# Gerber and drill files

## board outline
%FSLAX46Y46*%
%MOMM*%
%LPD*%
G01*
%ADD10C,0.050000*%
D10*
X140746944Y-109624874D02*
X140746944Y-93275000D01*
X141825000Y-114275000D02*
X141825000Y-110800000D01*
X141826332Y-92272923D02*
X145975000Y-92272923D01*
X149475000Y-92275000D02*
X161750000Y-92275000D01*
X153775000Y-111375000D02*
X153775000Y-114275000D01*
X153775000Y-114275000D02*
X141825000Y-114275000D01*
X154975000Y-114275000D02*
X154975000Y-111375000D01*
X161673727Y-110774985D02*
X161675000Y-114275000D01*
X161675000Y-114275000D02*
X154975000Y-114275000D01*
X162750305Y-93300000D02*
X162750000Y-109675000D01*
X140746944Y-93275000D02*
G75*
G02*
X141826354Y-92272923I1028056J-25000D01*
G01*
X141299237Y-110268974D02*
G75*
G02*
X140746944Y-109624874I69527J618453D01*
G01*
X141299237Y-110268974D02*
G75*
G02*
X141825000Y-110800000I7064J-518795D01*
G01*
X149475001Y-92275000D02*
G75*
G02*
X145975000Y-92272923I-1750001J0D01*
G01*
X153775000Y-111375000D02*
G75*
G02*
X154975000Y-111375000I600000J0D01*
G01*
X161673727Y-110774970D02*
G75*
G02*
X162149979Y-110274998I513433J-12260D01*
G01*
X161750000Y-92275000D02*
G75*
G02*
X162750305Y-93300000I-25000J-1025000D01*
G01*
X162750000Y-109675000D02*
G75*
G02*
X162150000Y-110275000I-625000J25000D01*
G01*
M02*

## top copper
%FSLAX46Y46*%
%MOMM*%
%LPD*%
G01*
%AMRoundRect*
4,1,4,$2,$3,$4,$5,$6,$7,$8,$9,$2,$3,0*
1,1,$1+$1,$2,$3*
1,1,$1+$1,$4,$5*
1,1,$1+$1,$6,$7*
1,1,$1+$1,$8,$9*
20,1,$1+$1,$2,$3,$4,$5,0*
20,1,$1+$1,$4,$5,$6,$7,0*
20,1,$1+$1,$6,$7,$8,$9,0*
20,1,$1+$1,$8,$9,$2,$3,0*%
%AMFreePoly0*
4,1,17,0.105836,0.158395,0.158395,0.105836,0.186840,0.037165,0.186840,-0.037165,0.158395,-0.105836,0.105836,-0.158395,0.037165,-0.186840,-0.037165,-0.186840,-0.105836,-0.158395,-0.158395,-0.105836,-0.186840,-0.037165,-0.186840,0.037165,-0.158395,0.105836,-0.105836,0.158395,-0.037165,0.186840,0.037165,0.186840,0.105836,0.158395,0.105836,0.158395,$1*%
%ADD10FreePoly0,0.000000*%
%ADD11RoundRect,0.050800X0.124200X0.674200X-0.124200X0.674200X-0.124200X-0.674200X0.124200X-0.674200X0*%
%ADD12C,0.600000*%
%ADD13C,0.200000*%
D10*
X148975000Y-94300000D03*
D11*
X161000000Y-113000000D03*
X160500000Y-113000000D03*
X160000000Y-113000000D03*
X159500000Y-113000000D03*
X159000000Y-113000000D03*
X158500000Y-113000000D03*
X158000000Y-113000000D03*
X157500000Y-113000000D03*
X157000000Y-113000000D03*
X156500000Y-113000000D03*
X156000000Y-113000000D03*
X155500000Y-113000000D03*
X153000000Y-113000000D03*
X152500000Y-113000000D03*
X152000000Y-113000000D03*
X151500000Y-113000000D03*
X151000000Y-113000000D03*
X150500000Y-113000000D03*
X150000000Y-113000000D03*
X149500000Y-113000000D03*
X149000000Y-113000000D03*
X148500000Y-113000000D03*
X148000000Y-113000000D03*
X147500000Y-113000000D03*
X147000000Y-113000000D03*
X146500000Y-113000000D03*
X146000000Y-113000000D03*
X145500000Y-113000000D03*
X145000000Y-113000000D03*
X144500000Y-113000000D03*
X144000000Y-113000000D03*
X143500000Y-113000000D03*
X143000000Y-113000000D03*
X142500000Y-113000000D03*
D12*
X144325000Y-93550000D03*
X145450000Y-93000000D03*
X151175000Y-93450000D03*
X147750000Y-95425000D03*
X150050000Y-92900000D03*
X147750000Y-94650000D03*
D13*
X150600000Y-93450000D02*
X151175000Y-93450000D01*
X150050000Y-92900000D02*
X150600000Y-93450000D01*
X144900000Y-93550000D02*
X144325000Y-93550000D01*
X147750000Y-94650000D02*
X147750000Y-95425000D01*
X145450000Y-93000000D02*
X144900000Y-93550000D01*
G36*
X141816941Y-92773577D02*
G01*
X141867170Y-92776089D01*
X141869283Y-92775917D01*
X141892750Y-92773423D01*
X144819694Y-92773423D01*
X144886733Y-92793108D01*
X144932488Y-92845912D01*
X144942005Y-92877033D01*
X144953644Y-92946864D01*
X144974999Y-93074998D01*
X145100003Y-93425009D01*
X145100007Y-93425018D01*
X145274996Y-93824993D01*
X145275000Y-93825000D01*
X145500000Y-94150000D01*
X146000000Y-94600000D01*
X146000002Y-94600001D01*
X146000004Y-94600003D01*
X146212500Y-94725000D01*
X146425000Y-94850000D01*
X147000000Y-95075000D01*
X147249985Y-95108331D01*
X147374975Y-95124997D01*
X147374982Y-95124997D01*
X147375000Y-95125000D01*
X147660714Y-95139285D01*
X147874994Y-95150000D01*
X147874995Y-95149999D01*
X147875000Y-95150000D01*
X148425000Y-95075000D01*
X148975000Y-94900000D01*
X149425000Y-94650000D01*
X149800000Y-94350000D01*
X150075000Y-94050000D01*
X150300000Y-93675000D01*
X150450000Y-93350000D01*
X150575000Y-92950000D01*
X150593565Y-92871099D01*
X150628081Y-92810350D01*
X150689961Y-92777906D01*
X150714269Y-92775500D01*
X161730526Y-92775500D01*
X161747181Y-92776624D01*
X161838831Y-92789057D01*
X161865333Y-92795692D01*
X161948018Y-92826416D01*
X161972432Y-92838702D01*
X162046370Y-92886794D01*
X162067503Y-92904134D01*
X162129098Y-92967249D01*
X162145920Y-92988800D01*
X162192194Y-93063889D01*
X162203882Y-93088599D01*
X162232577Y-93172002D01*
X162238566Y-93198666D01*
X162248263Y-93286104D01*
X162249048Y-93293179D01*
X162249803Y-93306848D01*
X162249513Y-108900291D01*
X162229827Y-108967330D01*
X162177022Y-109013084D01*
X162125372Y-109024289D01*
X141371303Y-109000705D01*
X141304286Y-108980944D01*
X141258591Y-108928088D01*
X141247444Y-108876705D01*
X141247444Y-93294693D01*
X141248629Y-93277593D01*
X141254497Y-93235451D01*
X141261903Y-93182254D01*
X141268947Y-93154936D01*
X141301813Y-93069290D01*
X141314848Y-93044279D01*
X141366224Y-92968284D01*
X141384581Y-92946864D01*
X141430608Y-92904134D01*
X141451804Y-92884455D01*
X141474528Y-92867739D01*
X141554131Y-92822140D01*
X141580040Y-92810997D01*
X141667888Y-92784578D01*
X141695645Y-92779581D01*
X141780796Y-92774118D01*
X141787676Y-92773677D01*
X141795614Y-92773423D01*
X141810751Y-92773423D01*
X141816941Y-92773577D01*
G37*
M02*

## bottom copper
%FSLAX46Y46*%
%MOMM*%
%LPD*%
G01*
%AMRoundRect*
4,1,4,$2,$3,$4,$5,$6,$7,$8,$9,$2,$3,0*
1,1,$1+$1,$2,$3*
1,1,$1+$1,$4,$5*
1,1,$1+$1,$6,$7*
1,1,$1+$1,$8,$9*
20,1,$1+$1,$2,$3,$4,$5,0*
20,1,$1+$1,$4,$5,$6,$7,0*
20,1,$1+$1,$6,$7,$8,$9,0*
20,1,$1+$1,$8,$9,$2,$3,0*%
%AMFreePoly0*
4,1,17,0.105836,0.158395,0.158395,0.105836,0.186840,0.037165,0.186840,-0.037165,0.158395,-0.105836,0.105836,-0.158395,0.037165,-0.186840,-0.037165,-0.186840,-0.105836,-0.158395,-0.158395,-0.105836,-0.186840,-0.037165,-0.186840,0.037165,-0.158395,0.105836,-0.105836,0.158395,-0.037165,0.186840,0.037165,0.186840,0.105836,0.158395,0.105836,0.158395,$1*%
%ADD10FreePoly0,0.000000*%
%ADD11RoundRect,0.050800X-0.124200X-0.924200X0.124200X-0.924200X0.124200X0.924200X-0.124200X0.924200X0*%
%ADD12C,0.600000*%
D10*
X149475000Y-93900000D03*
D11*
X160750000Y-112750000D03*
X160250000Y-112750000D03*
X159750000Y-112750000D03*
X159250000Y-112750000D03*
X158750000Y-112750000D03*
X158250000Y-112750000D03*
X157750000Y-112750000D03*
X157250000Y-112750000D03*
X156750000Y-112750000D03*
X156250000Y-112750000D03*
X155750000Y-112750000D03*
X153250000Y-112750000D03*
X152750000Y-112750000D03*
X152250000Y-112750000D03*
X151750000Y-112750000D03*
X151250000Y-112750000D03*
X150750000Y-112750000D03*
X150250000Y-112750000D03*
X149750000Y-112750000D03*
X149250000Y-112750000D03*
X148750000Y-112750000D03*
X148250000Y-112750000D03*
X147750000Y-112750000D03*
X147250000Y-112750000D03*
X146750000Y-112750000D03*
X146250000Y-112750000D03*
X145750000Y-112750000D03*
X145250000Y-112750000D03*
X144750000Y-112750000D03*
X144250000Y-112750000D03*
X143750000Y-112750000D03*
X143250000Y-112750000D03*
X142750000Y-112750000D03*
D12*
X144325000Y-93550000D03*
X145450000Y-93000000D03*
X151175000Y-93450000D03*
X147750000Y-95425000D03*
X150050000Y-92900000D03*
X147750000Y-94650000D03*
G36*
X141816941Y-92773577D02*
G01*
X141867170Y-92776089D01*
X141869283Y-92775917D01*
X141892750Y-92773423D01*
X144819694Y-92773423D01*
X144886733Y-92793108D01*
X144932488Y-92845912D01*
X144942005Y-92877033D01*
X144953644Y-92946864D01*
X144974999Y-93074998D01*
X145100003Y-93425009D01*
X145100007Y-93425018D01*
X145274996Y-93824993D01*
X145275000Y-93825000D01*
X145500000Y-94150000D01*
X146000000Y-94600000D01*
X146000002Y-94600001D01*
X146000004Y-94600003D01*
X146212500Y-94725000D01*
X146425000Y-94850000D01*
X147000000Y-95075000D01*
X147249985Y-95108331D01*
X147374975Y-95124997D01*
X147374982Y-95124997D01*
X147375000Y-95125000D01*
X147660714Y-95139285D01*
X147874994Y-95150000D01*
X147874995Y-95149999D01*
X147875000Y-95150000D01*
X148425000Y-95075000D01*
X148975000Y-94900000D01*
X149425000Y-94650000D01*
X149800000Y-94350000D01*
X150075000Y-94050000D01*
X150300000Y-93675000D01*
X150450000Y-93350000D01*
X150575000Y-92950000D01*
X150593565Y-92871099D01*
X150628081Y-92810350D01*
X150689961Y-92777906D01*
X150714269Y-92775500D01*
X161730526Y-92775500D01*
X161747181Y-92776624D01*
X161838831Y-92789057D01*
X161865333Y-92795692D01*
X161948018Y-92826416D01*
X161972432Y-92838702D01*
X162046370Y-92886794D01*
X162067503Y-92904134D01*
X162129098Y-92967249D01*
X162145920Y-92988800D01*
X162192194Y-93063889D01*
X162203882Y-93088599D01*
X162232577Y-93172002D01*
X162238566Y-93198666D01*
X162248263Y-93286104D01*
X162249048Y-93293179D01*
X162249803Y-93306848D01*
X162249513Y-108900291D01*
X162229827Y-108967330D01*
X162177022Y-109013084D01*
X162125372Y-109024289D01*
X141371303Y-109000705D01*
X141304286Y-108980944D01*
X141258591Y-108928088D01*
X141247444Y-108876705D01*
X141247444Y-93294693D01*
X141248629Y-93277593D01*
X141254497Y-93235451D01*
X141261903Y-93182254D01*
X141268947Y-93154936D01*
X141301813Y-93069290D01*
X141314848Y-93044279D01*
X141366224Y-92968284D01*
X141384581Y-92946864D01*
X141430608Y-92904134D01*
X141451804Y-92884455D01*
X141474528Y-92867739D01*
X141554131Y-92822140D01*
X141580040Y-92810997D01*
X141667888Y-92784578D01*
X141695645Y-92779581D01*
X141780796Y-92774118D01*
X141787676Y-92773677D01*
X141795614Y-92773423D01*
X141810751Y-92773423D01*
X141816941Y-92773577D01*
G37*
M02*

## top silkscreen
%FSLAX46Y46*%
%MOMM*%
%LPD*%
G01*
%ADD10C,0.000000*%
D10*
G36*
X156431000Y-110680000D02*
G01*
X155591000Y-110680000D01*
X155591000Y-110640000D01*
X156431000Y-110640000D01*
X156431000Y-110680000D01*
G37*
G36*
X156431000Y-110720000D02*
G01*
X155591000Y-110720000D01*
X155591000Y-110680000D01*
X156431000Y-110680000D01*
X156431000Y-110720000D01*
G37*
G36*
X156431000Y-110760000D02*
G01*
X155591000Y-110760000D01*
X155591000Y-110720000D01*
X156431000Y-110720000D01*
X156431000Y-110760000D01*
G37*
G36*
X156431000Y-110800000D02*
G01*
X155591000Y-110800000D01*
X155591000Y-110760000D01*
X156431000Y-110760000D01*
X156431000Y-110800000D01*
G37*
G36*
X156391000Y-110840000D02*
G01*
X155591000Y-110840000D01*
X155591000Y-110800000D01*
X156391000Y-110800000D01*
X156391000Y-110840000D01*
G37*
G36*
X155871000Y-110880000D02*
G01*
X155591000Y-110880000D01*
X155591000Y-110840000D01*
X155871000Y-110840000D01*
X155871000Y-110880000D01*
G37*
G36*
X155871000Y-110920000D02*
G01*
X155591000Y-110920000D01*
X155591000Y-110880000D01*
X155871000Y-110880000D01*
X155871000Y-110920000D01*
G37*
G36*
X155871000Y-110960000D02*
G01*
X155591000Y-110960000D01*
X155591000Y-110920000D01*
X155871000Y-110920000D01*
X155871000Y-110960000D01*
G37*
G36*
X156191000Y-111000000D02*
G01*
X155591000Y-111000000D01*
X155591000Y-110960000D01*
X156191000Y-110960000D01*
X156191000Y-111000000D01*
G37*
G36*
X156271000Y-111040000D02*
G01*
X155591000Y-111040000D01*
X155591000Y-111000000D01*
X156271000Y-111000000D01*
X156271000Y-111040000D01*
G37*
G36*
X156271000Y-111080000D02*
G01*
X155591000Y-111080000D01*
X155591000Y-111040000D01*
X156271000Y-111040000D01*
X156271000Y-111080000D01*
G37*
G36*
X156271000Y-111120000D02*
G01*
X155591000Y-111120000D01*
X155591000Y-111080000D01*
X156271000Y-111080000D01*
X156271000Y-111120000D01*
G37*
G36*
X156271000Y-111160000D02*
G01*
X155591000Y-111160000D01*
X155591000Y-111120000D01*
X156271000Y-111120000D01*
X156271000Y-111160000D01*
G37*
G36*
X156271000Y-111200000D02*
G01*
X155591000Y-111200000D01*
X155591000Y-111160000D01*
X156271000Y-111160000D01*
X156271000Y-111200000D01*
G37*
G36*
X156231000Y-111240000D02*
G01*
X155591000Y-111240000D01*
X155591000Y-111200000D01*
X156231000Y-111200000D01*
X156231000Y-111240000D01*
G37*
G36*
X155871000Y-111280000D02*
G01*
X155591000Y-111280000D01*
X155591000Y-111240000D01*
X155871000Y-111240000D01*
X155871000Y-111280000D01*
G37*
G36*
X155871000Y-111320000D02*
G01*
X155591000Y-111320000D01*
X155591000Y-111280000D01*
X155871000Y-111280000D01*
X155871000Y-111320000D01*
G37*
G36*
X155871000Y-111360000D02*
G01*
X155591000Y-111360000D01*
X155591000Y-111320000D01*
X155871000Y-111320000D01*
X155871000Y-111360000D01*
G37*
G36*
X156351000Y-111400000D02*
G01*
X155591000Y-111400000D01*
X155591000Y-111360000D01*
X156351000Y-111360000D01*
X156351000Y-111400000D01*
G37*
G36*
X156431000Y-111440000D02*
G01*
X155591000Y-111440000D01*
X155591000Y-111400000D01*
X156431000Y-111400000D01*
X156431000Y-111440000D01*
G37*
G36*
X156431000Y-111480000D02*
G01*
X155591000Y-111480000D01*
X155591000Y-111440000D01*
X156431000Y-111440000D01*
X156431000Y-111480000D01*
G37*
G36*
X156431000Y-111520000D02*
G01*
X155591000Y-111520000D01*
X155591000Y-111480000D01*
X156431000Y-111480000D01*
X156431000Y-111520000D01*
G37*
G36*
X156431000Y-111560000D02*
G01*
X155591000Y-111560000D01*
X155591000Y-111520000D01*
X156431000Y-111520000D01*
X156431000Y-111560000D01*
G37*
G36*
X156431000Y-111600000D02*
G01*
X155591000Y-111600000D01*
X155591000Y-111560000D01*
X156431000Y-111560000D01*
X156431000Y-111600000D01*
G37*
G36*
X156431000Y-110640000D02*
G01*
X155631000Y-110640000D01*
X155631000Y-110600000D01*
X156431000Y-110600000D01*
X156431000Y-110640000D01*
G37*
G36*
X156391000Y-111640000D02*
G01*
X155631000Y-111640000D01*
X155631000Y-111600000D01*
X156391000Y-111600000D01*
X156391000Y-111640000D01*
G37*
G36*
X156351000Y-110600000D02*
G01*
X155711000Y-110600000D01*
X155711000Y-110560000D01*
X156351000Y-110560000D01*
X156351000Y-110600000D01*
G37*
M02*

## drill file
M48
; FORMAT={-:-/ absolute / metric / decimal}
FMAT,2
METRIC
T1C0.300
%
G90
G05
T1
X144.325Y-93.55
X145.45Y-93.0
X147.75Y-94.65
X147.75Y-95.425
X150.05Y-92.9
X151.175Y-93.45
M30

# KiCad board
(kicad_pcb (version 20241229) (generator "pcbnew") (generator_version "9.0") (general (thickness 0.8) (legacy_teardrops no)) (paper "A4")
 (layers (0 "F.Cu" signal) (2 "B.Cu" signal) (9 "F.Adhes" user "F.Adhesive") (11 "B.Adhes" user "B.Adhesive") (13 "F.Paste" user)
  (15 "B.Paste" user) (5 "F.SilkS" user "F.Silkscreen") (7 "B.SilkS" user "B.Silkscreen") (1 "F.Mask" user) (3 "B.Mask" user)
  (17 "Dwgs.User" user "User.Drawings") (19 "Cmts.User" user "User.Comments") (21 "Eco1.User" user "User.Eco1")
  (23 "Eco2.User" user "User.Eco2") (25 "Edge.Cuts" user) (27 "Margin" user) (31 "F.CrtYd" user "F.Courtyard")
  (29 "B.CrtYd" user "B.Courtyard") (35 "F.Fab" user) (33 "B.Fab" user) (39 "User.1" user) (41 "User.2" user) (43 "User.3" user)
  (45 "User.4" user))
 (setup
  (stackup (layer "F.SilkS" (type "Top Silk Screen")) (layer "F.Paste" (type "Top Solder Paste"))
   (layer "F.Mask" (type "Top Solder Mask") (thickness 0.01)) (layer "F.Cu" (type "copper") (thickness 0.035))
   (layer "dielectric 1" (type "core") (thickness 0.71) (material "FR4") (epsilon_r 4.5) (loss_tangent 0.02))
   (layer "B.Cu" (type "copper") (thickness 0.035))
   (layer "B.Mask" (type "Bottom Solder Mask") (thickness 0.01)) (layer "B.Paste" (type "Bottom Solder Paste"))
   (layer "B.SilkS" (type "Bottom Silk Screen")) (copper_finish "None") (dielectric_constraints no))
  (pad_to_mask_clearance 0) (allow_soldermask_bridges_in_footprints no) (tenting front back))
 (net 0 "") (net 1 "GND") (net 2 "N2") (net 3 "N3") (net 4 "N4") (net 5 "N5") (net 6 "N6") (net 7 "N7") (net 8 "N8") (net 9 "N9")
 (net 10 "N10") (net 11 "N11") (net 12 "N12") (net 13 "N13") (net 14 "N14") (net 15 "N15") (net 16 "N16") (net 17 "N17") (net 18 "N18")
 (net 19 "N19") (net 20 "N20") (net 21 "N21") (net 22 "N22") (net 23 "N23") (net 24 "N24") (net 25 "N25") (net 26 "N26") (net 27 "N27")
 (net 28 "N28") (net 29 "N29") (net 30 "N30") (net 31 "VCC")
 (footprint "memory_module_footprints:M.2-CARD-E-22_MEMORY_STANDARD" (layer "F.Cu") (at 151.75 114.275)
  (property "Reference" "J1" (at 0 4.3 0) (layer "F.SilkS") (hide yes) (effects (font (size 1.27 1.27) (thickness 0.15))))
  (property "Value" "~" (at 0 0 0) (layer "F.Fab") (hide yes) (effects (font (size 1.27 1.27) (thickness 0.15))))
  (fp_poly
   (pts (xy 3.841 -3.595) (xy 4.681 -3.595) (xy 4.681 -3.635) (xy 3.841 -3.635)) (stroke (width 0) (type default)) (fill yes)
   (layer "F.SilkS"))
  (fp_poly
   (pts (xy 3.841 -3.555) (xy 4.681 -3.555) (xy 4.681 -3.595) (xy 3.841 -3.595)) (stroke (width 0) (type default)) (fill yes)
   (layer "F.SilkS"))
  (fp_poly
   (pts (xy 3.841 -3.515) (xy 4.681 -3.515) (xy 4.681 -3.555) (xy 3.841 -3.555)) (stroke (width 0) (type default)) (fill yes)
   (layer "F.SilkS"))
  (fp_poly
   (pts (xy 3.841 -3.475) (xy 4.681 -3.475) (xy 4.681 -3.515) (xy 3.841 -3.515)) (stroke (width 0) (type default)) (fill yes)
   (layer "F.SilkS"))
  (fp_poly
   (pts (xy 3.841 -3.435) (xy 4.641 -3.435) (xy 4.641 -3.475) (xy 3.841 -3.475)) (stroke (width 0) (type default)) (fill yes)
   (layer "F.SilkS"))
  (fp_poly
   (pts (xy 3.841 -3.395) (xy 4.121 -3.395) (xy 4.121 -3.435) (xy 3.841 -3.435)) (stroke (width 0) (type default)) (fill yes)
   (layer "F.SilkS"))
  (fp_poly
   (pts (xy 3.841 -3.355) (xy 4.121 -3.355) (xy 4.121 -3.395) (xy 3.841 -3.395)) (stroke (width 0) (type default)) (fill yes)
   (layer "F.SilkS"))
  (fp_poly
   (pts (xy 3.841 -3.315) (xy 4.121 -3.315) (xy 4.121 -3.355) (xy 3.841 -3.355)) (stroke (width 0) (type default)) (fill yes)
   (layer "F.SilkS"))
  (fp_poly
   (pts (xy 3.841 -3.275) (xy 4.441 -3.275) (xy 4.441 -3.315) (xy 3.841 -3.315)) (stroke (width 0) (type default)) (fill yes)
   (layer "F.SilkS"))
  (fp_poly
   (pts (xy 3.841 -3.235) (xy 4.521 -3.235) (xy 4.521 -3.275) (xy 3.841 -3.275)) (stroke (width 0) (type default)) (fill yes)
   (layer "F.SilkS"))
  (fp_poly
   (pts (xy 3.841 -3.195) (xy 4.521 -3.195) (xy 4.521 -3.235) (xy 3.841 -3.235)) (stroke (width 0) (type default)) (fill yes)
   (layer "F.SilkS"))
  (fp_poly
   (pts (xy 3.841 -3.155) (xy 4.521 -3.155) (xy 4.521 -3.195) (xy 3.841 -3.195)) (stroke (width 0) (type default)) (fill yes)
   (layer "F.SilkS"))
  (fp_poly
   (pts (xy 3.841 -3.115) (xy 4.521 -3.115) (xy 4.521 -3.155) (xy 3.841 -3.155)) (stroke (width 0) (type default)) (fill yes)
   (layer "F.SilkS"))
  (fp_poly
   (pts (xy 3.841 -3.075) (xy 4.521 -3.075) (xy 4.521 -3.115) (xy 3.841 -3.115)) (stroke (width 0) (type default)) (fill yes)
   (layer "F.SilkS"))
  (fp_poly
   (pts (xy 3.841 -3.035) (xy 4.481 -3.035) (xy 4.481 -3.075) (xy 3.841 -3.075)) (stroke (width 0) (type default)) (fill yes)
   (layer "F.SilkS"))
  (fp_poly
   (pts (xy 3.841 -2.995) (xy 4.121 -2.995) (xy 4.121 -3.035) (xy 3.841 -3.035)) (stroke (width 0) (type default)) (fill yes)
   (layer "F.SilkS"))
  (fp_poly
   (pts (xy 3.841 -2.955) (xy 4.121 -2.955) (xy 4.121 -2.995) (xy 3.841 -2.995)) (stroke (width 0) (type default)) (fill yes)
   (layer "F.SilkS"))
  (fp_poly
   (pts (xy 3.841 -2.915) (xy 4.121 -2.915) (xy 4.121 -2.955) (xy 3.841 -2.955)) (stroke (width 0) (type default)) (fill yes)
   (layer "F.SilkS"))
  (fp_poly
   (pts (xy 3.841 -2.875) (xy 4.601 -2.875) (xy 4.601 -2.915) (xy 3.841 -2.915)) (stroke (width 0) (type default)) (fill yes)
   (layer "F.SilkS"))
  (fp_poly
   (pts (xy 3.841 -2.835) (xy 4.681 -2.835) (xy 4.681 -2.875) (xy 3.841 -2.875)) (stroke (width 0) (type default)) (fill yes)
   (layer "F.SilkS"))
  (fp_poly
   (pts (xy 3.841 -2.795) (xy 4.681 -2.795) (xy 4.681 -2.835) (xy 3.841 -2.835)) (stroke (width 0) (type default)) (fill yes)
   (layer "F.SilkS"))
  (fp_poly
   (pts (xy 3.841 -2.755) (xy 4.681 -2.755) (xy 4.681 -2.795) (xy 3.841 -2.795)) (stroke (width 0) (type default)) (fill yes)
   (layer "F.SilkS"))
  (fp_poly
   (pts (xy 3.841 -2.715) (xy 4.681 -2.715) (xy 4.681 -2.755) (xy 3.841 -2.755)) (stroke (width 0) (type default)) (fill yes)
   (layer "F.SilkS"))
  (fp_poly
   (pts (xy 3.841 -2.675) (xy 4.681 -2.675) (xy 4.681 -2.715) (xy 3.841 -2.715)) (stroke (width 0) (type default)) (fill yes)
   (layer "F.SilkS"))
  (fp_poly
   (pts (xy 3.881 -3.635) (xy 4.681 -3.635) (xy 4.681 -3.675) (xy 3.881 -3.675)) (stroke (width 0) (type default)) (fill yes)
   (layer "F.SilkS"))
  (fp_poly
   (pts (xy 3.881 -2.635) (xy 4.641 -2.635) (xy 4.641 -2.675) (xy 3.881 -2.675)) (stroke (width 0) (type default)) (fill yes)
   (layer "F.SilkS"))
  (fp_poly
   (pts (xy 3.961 -3.675) (xy 4.601 -3.675) (xy 4.601 -3.715) (xy 3.961 -3.715)) (stroke (width 0) (type default)) (fill yes)
   (layer "F.SilkS"))
  (fp_line (start -11.003056 -4.650126) (end -11.003056 -21) (stroke (width 0.05) (type default)) (layer "Edge.Cuts"))
  (fp_line (start -9.925 0) (end -9.925 -3.475) (stroke (width 0.05) (type default)) (layer "Edge.Cuts"))
  (fp_line (start -9.923668 -22.002077) (end -5.775 -22.002077) (stroke (width 0.05) (type default)) (layer "Edge.Cuts"))
  (fp_line (start -2.275 -22) (end 10 -22) (stroke (width 0.05) (type default)) (layer "Edge.Cuts"))
  (fp_line (start 2.025 -2.9) (end 2.025 0) (stroke (width 0.05) (type default)) (layer "Edge.Cuts"))
  (fp_line (start 2.025 0) (end -9.925 0) (stroke (width 0.05) (type default)) (layer "Edge.Cuts"))
  (fp_line (start 3.225 0) (end 3.225 -2.9) (stroke (width 0.05) (type default)) (layer "Edge.Cuts"))
  (fp_line (start 9.923727 -3.500015) (end 9.925 0) (stroke (width 0.05) (type default)) (layer "Edge.Cuts"))
  (fp_line (start 9.925 0) (end 3.225 0) (stroke (width 0.05) (type default)) (layer "Edge.Cuts"))
  (fp_line (start 11.000305 -20.975) (end 11 -4.6) (stroke (width 0.05) (type default)) (layer "Edge.Cuts"))
  (fp_arc (start -11.003056 -21) (mid -10.674662 -21.728656) (end -9.923646 -22.002077) (stroke (width 0.05) (type default))
   (layer "Edge.Cuts"))
  (fp_arc (start -10.450763 -4.006026) (mid -10.853683 -4.219372) (end -11.003056 -4.650126) (stroke (width 0.05) (type default))
   (layer "Edge.Cuts"))
  (fp_arc (start -10.450763 -4.006026) (mid -10.074999 -3.852277) (end -9.925 -3.475) (stroke (width 0.05) (type default))
   (layer "Edge.Cuts"))
  (fp_arc (start -2.274999 -22) (mid -4.026039 -20.249999) (end -5.775 -22.002077) (stroke (width 0.05) (type default)) (layer "Edge.Cuts"))
  (fp_arc (start 2.025 -2.9) (mid 2.625 -3.5) (end 3.225 -2.9) (stroke (width 0.05) (type default)) (layer "Edge.Cuts"))
  (fp_arc (start 9.923727 -3.50003) (mid 10.065291 -3.841996) (end 10.399979 -4) (stroke (width 0.05) (type default)) (layer "Edge.Cuts"))
  (fp_arc (start 10 -22) (mid 10.708786 -21.691107) (end 11.000305 -20.975) (stroke (width 0.05) (type default)) (layer "Edge.Cuts"))
  (fp_arc (start 11 -4.6) (mid 10.817295 -4.182705) (end 10.4 -4) (stroke (width 0.05) (type default)) (layer "Edge.Cuts"))
  (pad "1" smd custom (at -2.775 -19.975) (size 0.381 0.381) (layers "F.Cu") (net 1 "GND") (solder_mask_margin 0.0635)
   (thermal_bridge_angle 0) (options (clearance outline) (anchor circle)) (primitives))
  (pad "1" smd custom (at -2.275 -20.375) (size 0.381 0.381) (layers "B.Cu") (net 1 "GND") (solder_mask_margin 0.0635)
   (thermal_bridge_angle 0) (options (clearance outline) (anchor circle)) (primitives))
  (pad "1" smd roundrect (at 9.25 -1.275 180) (size 0.35 1.45) (layers "F.Cu" "F.Mask") (roundrect_rratio 0.1451428571) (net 1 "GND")
   (solder_mask_margin 0.0635) (solder_paste_margin 0) (thermal_bridge_angle 0))
  (pad "2" smd roundrect (at 9 -1.525) (size 0.35 1.95) (layers "B.Cu" "B.Mask") (roundrect_rratio 0.1451428571) (solder_mask_margin 0.0635)
   (solder_paste_margin 0) (thermal_bridge_angle 0))
  (pad "3" smd roundrect (at 8.75 -1.275 180) (size 0.35 1.45) (layers "F.Cu" "F.Mask") (roundrect_rratio 0.1451428571) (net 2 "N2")
   (solder_mask_margin 0.0635) (solder_paste_margin 0) (thermal_bridge_angle 0))
  (pad "4" smd roundrect (at 8.5 -1.525) (size 0.35 1.95) (layers "B.Cu" "B.Mask") (roundrect_rratio 0.1451428571)
   (solder_mask_margin 0.0635) (solder_paste_margin 0) (thermal_bridge_angle 0))
  (pad "5" smd roundrect (at 8.25 -1.275 180) (size 0.35 1.45) (layers "F.Cu" "F.Mask") (roundrect_rratio 0.1451428571) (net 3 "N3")
   (solder_mask_margin 0.0635) (solder_paste_margin 0) (thermal_bridge_angle 0))
  (pad "6" smd roundrect (at 8 -1.525) (size 0.35 1.95) (layers "B.Cu" "B.Mask") (roundrect_rratio 0.1451428571) (solder_mask_margin 0.0635)
   (solder_paste_margin 0) (thermal_bridge_angle 0))
  (pad "7" smd roundrect (at 7.75 -1.275 180) (size 0.35 1.45) (layers "F.Cu" "F.Mask") (roundrect_rratio 0.1451428571) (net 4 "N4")
   (solder_mask_margin 0.0635) (solder_paste_margin 0) (thermal_bridge_angle 0))
  (pad "8" smd roundrect (at 7.5 -1.525) (size 0.35 1.95) (layers "B.Cu" "B.Mask") (roundrect_rratio 0.1451428571)
   (solder_mask_margin 0.0635) (solder_paste_margin 0) (thermal_bridge_angle 0))
  (pad "9" smd roundrect (at 7.25 -1.275 180) (size 0.35 1.45) (layers "F.Cu" "F.Mask") (roundrect_rratio 0.1451428571)
   (solder_mask_margin 0.0635) (solder_paste_margin 0) (thermal_bridge_angle 0))
  (pad "10" smd roundrect (at 7 -1.525) (size 0.35 1.95) (layers "B.Cu" "B.Mask") (roundrect_rratio 0.1451428571)
   (solder_mask_margin 0.0635) (solder_paste_margin 0) (thermal_bridge_angle 0))
  (pad "11" smd roundrect (at 6.75 -1.275 180) (size 0.35 1.45) (layers "F.Cu" "F.Mask") (roundrect_rratio 0.1451428571)
   (solder_mask_margin 0.0635) (solder_paste_margin 0) (thermal_bridge_angle 0))
  (pad "12" smd roundrect (at 6.5 -1.525) (size 0.35 1.95) (layers "B.Cu" "B.Mask") (roundrect_rratio 0.1451428571)
   (solder_mask_margin 0.0635) (solder_paste_margin 0) (thermal_bridge_angle 0))
  (pad "13" smd roundrect (at 6.25 -1.275 180) (size 0.35 1.45) (layers "F.Cu" "F.Mask") (roundrect_rratio 0.1451428571) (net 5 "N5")
   (solder_mask_margin 0.0635) (solder_paste_margin 0) (thermal_bridge_angle 0))
  (pad "14" smd roundrect (at 6 -1.525) (size 0.35 1.95) (layers "B.Cu" "B.Mask") (roundrect_rratio 0.1451428571)
   (solder_mask_margin 0.0635) (solder_paste_margin 0) (thermal_bridge_angle 0))
  (pad "15" smd roundrect (at 5.75 -1.275 180) (size 0.35 1.45) (layers "F.Cu" "F.Mask") (roundrect_rratio 0.1451428571) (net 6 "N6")
   (solder_mask_margin 0.0635) (solder_paste_margin 0) (thermal_bridge_angle 0))
  (pad "16" smd roundrect (at 5.5 -1.525) (size 0.35 1.95) (layers "B.Cu" "B.Mask") (roundrect_rratio 0.1451428571) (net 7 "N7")
   (solder_mask_margin 0.0635) (solder_paste_margin 0) (thermal_bridge_angle 0))
  (pad "17" smd roundrect (at 5.25 -1.275 180) (size 0.35 1.45) (layers "F.Cu" "F.Mask") (roundrect_rratio 0.1451428571)
   (solder_mask_margin 0.0635) (solder_paste_margin 0) (thermal_bridge_angle 0))
  (pad "18" smd roundrect (at 5 -1.525) (size 0.35 1.95) (layers "B.Cu" "B.Mask") (roundrect_rratio 0.1451428571) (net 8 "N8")
   (solder_mask_margin 0.0635) (solder_paste_margin 0) (thermal_bridge_angle 0))
  (pad "19" smd roundrect (at 4.75 -1.275 180) (size 0.35 1.45) (layers "F.Cu" "F.Mask") (roundrect_rratio 0.1451428571) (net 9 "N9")
   (solder_mask_margin 0.0635) (solder_paste_margin 0) (thermal_bridge_angle 0))
  (pad "20" smd roundrect (at 4.5 -1.525) (size 0.35 1.95) (layers "B.Cu" "B.Mask") (roundrect_rratio 0.1451428571)
   (solder_mask_margin 0.0635) (solder_paste_margin 0) (thermal_bridge_angle 0))
  (pad "21" smd roundrect (at 4.25 -1.275 180) (size 0.35 1.45) (layers "F.Cu" "F.Mask") (roundrect_rratio 0.1451428571) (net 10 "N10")
   (solder_mask_margin 0.0635) (solder_paste_margin 0) (thermal_bridge_angle 0))
  (pad "22" smd roundrect (at 4 -1.525) (size 0.35 1.95) (layers "B.Cu" "B.Mask") (roundrect_rratio 0.1451428571)
   (solder_mask_margin 0.0635) (solder_paste_margin 0) (thermal_bridge_angle 0))
  (pad "23" smd roundrect (at 3.75 -1.275 180) (size 0.35 1.45) (layers "F.Cu" "F.Mask") (roundrect_rratio 0.1451428571) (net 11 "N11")
   (solder_mask_margin 0.0635) (solder_paste_margin 0) (thermal_bridge_angle 0))
  (pad "32" smd roundrect (at 1.5 -1.525) (size 0.35 1.95) (layers "B.Cu" "B.Mask") (roundrect_rratio 0.1451428571) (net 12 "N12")
   (solder_mask_margin 0.0635) (solder_paste_margin 0) (thermal_bridge_angle 0))
  (pad "33" smd roundrect (at 1.25 -1.275 180) (size 0.35 1.45) (layers "F.Cu" "F.Mask") (roundrect_rratio 0.1451428571) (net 1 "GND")
   (solder_mask_margin 0.0635) (solder_paste_margin 0) (thermal_bridge_angle 0))
  (pad "34" smd roundrect (at 1 -1.525) (size 0.35 1.95) (layers "B.Cu" "B.Mask") (roundrect_rratio 0.1451428571) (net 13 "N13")
   (solder_mask_margin 0.0635) (solder_paste_margin 0) (thermal_bridge_angle 0))
  (pad "35" smd roundrect (at 0.75 -1.275 180) (size 0.35 1.45) (layers "F.Cu" "F.Mask") (roundrect_rratio 0.1451428571) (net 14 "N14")
   (solder_mask_margin 0.0635) (solder_paste_margin 0) (thermal_bridge_angle 0))
  (pad "36" smd roundrect (at 0.5 -1.525) (size 0.35 1.95) (layers "B.Cu" "B.Mask") (roundrect_rratio 0.1451428571) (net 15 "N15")
   (solder_mask_margin 0.0635) (solder_paste_margin 0) (thermal_bridge_angle 0))
  (pad "37" smd roundrect (at 0.25 -1.275 180) (size 0.35 1.45) (layers "F.Cu" "F.Mask") (roundrect_rratio 0.1451428571) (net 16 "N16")
   (solder_mask_margin 0.0635) (solder_paste_margin 0) (thermal_bridge_angle 0))
  (pad "38" smd roundrect (at 0 -1.525) (size 0.35 1.95) (layers "B.Cu" "B.Mask") (roundrect_rratio 0.1451428571) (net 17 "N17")
   (solder_mask_margin 0.0635) (solder_paste_margin 0) (thermal_bridge_angle 0))
  (pad "39" smd roundrect (at -0.25 -1.275 180) (size 0.35 1.45) (layers "F.Cu" "F.Mask") (roundrect_rratio 0.1451428571) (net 1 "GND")
   (solder_mask_margin 0.0635) (solder_paste_margin 0) (thermal_bridge_angle 0))
  (pad "40" smd roundrect (at -0.5 -1.525) (size 0.35 1.95) (layers "B.Cu" "B.Mask") (roundrect_rratio 0.1451428571)
   (solder_mask_margin 0.0635) (solder_paste_margin 0) (thermal_bridge_angle 0))
  (pad "41" smd roundrect (at -0.75 -1.275 180) (size 0.35 1.45) (layers "F.Cu" "F.Mask") (roundrect_rratio 0.1451428571) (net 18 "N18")
   (solder_mask_margin 0.0635) (solder_paste_margin 0) (thermal_bridge_angle 0))
  (pad "42" smd roundrect (at -1 -1.525) (size 0.35 1.95) (layers "B.Cu" "B.Mask") (roundrect_rratio 0.1451428571)
   (solder_mask_margin 0.0635) (solder_paste_margin 0) (thermal_bridge_angle 0))
  (pad "43" smd roundrect (at -1.25 -1.275 180) (size 0.35 1.45) (layers "F.Cu" "F.Mask") (roundrect_rratio 0.1451428571) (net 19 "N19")
   (solder_mask_margin 0.0635) (solder_paste_margin 0) (thermal_bridge_angle 0))
  (pad "44" smd roundrect (at -1.5 -1.525) (size 0.35 1.95) (layers "B.Cu" "B.Mask") (roundrect_rratio 0.1451428571)
   (solder_mask_margin 0.0635) (solder_paste_margin 0) (thermal_bridge_angle 0))
  (pad "45" smd roundrect (at -1.75 -1.275 180) (size 0.35 1.45) (layers "F.Cu" "F.Mask") (roundrect_rratio 0.1451428571) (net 1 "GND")
   (solder_mask_margin 0.0635) (solder_paste_margin 0) (thermal_bridge_angle 0))
  (pad "46" smd roundrect (at -2 -1.525) (size 0.35 1.95) (layers "B.Cu" "B.Mask") (roundrect_rratio 0.1451428571)
   (solder_mask_margin 0.0635) (solder_paste_margin 0) (thermal_bridge_angle 0))
  (pad "47" smd roundrect (at -2.25 -1.275 180) (size 0.35 1.45) (layers "F.Cu" "F.Mask") (roundrect_rratio 0.1451428571) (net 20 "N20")
   (solder_mask_margin 0.0635) (solder_paste_margin 0) (thermal_bridge_angle 0))
  (pad "48" smd roundrect (at -2.5 -1.525) (size 0.35 1.95) (layers "B.Cu" "B.Mask") (roundrect_rratio 0.1451428571)
   (solder_mask_margin 0.0635) (solder_paste_margin 0) (thermal_bridge_angle 0))
  (pad "49" smd roundrect (at -2.75 -1.275 180) (size 0.35 1.45) (layers "F.Cu" "F.Mask") (roundrect_rratio 0.1451428571) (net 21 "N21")
   (solder_mask_margin 0.0635) (solder_paste_margin 0) (thermal_bridge_angle 0))
  (pad "50" smd roundrect (at -3 -1.525) (size 0.35 1.95) (layers "B.Cu" "B.Mask") (roundrect_rratio 0.1451428571)
   (solder_mask_margin 0.0635) (solder_paste_margin 0) (thermal_bridge_angle 0))
  (pad "51" smd roundrect (at -3.25 -1.275 180) (size 0.35 1.45) (layers "F.Cu" "F.Mask") (roundrect_rratio 0.1451428571) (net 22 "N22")
   (solder_mask_margin 0.0635) (solder_paste_margin 0) (thermal_bridge_angle 0))
  (pad "52" smd roundrect (at -3.5 -1.525) (size 0.35 1.95) (layers "B.Cu" "B.Mask") (roundrect_rratio 0.1451428571)
   (solder_mask_margin 0.0635) (solder_paste_margin 0) (thermal_bridge_angle 0))
  (pad "53" smd roundrect (at -3.75 -1.275 180) (size 0.35 1.45) (layers "F.Cu" "F.Mask") (roundrect_rratio 0.1451428571) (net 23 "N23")
   (solder_mask_margin 0.0635) (solder_paste_margin 0) (thermal_bridge_angle 0))
  (pad "54" smd roundrect (at -4 -1.525) (size 0.35 1.95) (layers "B.Cu" "B.Mask") (roundrect_rratio 0.1451428571)
   (solder_mask_margin 0.0635) (solder_paste_margin 0) (thermal_bridge_angle 0))
  (pad "55" smd roundrect (at -4.25 -1.275 180) (size 0.35 1.45) (layers "F.Cu" "F.Mask") (roundrect_rratio 0.1451428571) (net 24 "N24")
   (solder_mask_margin 0.0635) (solder_paste_margin 0) (thermal_bridge_angle 0))
  (pad "56" smd roundrect (at -4.5 -1.525) (size 0.35 1.95) (layers "B.Cu" "B.Mask") (roundrect_rratio 0.1451428571)
   (solder_mask_margin 0.0635) (solder_paste_margin 0) (thermal_bridge_angle 0))
  (pad "57" smd roundrect (at -4.75 -1.275 180) (size 0.35 1.45) (layers "F.Cu" "F.Mask") (roundrect_rratio 0.1451428571) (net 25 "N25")
   (solder_mask_margin 0.0635) (solder_paste_margin 0) (thermal_bridge_angle 0))
  (pad "58" smd roundrect (at -5 -1.525) (size 0.35 1.95) (layers "B.Cu" "B.Mask") (roundrect_rratio 0.1451428571)
   (solder_mask_margin 0.0635) (solder_paste_margin 0) (thermal_bridge_angle 0))
  (pad "59" smd roundrect (at -5.25 -1.275 180) (size 0.35 1.45) (layers "F.Cu" "F.Mask") (roundrect_rratio 0.1451428571) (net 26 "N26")
   (solder_mask_margin 0.0635) (solder_paste_margin 0) (thermal_bridge_angle 0))
  (pad "60" smd roundrect (at -5.5 -1.525) (size 0.35 1.95) (layers "B.Cu" "B.Mask") (roundrect_rratio 0.1451428571)
   (solder_mask_margin 0.0635) (solder_paste_margin 0) (thermal_bridge_angle 0))
  (pad "61" smd roundrect (at -5.75 -1.275 180) (size 0.35 1.45) (layers "F.Cu" "F.Mask") (roundrect_rratio 0.1451428571) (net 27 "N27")
   (solder_mask_margin 0.0635) (solder_paste_margin 0) (thermal_bridge_angle 0))
  (pad "62" smd roundrect (at -6 -1.525) (size 0.35 1.95) (layers "B.Cu" "B.Mask") (roundrect_rratio 0.1451428571)
   (solder_mask_margin 0.0635) (solder_paste_margin 0) (thermal_bridge_angle 0))
  (pad "63" smd roundrect (at -6.25 -1.275 180) (size 0.35 1.45) (layers "F.Cu" "F.Mask") (roundrect_rratio 0.1451428571)
   (solder_mask_margin 0.0635) (solder_paste_margin 0) (thermal_bridge_angle 0))
  (pad "64" smd roundrect (at -6.5 -1.525) (size 0.35 1.95) (layers "B.Cu" "B.Mask") (roundrect_rratio 0.1451428571)
   (solder_mask_margin 0.0635) (solder_paste_margin 0) (thermal_bridge_angle 0))
  (pad "65" smd roundrect (at -6.75 -1.275 180) (size 0.35 1.45) (layers "F.Cu" "F.Mask") (roundrect_rratio 0.1451428571)
   (solder_mask_margin 0.0635) (solder_paste_margin 0) (thermal_bridge_angle 0))
  (pad "66" smd roundrect (at -7 -1.525) (size 0.35 1.95) (layers "B.Cu" "B.Mask") (roundrect_rratio 0.1451428571)
   (solder_mask_margin 0.0635) (solder_paste_margin 0) (thermal_bridge_angle 0))
  (pad "67" smd roundrect (at -7.25 -1.275 180) (size 0.35 1.45) (layers "F.Cu" "F.Mask") (roundrect_rratio 0.1451428571)
   (solder_mask_margin 0.0635) (solder_paste_margin 0) (thermal_bridge_angle 0))
  (pad "68" smd roundrect (at -7.5 -1.525) (size 0.35 1.95) (layers "B.Cu" "B.Mask") (roundrect_rratio 0.1451428571)
   (solder_mask_margin 0.0635) (solder_paste_margin 0) (thermal_bridge_angle 0))
  (pad "69" smd roundrect (at -7.75 -1.275 180) (size 0.35 1.45) (layers "F.Cu" "F.Mask") (roundrect_rratio 0.1451428571)
   (solder_mask_margin 0.0635) (solder_paste_margin 0) (thermal_bridge_angle 0))
  (pad "70" smd roundrect (at -8 -1.525) (size 0.35 1.95) (layers "B.Cu" "B.Mask") (roundrect_rratio 0.1451428571) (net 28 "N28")
   (solder_mask_margin 0.0635) (solder_paste_margin 0) (thermal_bridge_angle 0))
  (pad "71" smd roundrect (at -8.25 -1.275 180) (size 0.35 1.45) (layers "F.Cu" "F.Mask") (roundrect_rratio 0.1451428571) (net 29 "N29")
   (solder_mask_margin 0.0635) (solder_paste_margin 0) (thermal_bridge_angle 0))
  (pad "72" smd roundrect (at -8.5 -1.525) (size 0.35 1.95) (layers "B.Cu" "B.Mask") (roundrect_rratio 0.1451428571) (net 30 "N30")
   (solder_mask_margin 0.0635) (solder_paste_margin 0) (thermal_bridge_angle 0))
  (pad "73" smd roundrect (at -8.75 -1.275 180) (size 0.35 1.45) (layers "F.Cu" "F.Mask") (roundrect_rratio 0.1451428571) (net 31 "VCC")
   (solder_mask_margin 0.0635) (solder_paste_margin 0) (thermal_bridge_angle 0))
  (pad "74" smd roundrect (at -9 -1.525) (size 0.35 1.95) (layers "B.Cu" "B.Mask") (roundrect_rratio 0.1451428571) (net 30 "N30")
   (solder_mask_margin 0.0635) (solder_paste_margin 0) (thermal_bridge_angle 0))
  (pad "75" smd roundrect (at -9.25 -1.275 180) (size 0.35 1.45) (layers "F.Cu" "F.Mask") (roundrect_rratio 0.1451428571) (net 1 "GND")
   (solder_mask_margin 0.0635) (solder_paste_margin 0) (thermal_bridge_angle 0)))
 (segment (start 150.6 93.45) (end 151.175 93.45) (width 0.2) (layer "F.Cu") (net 1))
 (segment (start 150.05 92.9) (end 150.6 93.45) (width 0.2) (layer "F.Cu") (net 1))
 (segment (start 144.9 93.55) (end 144.325 93.55) (width 0.2) (layer "F.Cu") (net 1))
 (segment (start 147.75 94.65) (end 147.75 95.425) (width 0.2) (layer "F.Cu") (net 1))
 (segment (start 145.45 93) (end 144.9 93.55) (width 0.2) (layer "F.Cu") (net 1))
 (via (at 144.325 93.55) (size 0.6) (drill 0.3) (layers "F.Cu" "B.Cu") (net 1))
 (via (at 145.45 93) (size 0.6) (drill 0.3) (layers "F.Cu" "B.Cu") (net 1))
 (via (at 151.175 93.45) (size 0.6) (drill 0.3) (layers "F.Cu" "B.Cu") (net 1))
 (via (at 147.75 95.425) (size 0.6) (drill 0.3) (layers "F.Cu" "B.Cu") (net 1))
 (via (at 150.05 92.9) (size 0.6) (drill 0.3) (layers "F.Cu" "B.Cu") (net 1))
 (via (at 147.75 94.65) (size 0.6) (drill 0.3) (layers "F.Cu" "B.Cu") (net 1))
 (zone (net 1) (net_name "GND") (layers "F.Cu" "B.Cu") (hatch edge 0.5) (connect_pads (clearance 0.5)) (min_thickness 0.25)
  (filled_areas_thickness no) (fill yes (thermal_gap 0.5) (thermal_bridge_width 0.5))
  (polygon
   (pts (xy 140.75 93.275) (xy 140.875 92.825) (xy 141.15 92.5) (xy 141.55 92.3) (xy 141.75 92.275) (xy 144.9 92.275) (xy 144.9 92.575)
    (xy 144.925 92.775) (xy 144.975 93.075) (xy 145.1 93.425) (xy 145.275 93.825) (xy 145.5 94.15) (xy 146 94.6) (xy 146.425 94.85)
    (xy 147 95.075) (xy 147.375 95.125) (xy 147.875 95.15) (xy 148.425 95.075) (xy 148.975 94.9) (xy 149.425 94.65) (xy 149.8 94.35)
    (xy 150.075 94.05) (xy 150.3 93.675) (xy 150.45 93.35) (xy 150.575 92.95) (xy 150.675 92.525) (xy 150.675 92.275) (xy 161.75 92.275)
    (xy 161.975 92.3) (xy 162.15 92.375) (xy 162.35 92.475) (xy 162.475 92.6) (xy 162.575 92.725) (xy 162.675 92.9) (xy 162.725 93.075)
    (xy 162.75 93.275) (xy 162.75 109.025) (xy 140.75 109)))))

